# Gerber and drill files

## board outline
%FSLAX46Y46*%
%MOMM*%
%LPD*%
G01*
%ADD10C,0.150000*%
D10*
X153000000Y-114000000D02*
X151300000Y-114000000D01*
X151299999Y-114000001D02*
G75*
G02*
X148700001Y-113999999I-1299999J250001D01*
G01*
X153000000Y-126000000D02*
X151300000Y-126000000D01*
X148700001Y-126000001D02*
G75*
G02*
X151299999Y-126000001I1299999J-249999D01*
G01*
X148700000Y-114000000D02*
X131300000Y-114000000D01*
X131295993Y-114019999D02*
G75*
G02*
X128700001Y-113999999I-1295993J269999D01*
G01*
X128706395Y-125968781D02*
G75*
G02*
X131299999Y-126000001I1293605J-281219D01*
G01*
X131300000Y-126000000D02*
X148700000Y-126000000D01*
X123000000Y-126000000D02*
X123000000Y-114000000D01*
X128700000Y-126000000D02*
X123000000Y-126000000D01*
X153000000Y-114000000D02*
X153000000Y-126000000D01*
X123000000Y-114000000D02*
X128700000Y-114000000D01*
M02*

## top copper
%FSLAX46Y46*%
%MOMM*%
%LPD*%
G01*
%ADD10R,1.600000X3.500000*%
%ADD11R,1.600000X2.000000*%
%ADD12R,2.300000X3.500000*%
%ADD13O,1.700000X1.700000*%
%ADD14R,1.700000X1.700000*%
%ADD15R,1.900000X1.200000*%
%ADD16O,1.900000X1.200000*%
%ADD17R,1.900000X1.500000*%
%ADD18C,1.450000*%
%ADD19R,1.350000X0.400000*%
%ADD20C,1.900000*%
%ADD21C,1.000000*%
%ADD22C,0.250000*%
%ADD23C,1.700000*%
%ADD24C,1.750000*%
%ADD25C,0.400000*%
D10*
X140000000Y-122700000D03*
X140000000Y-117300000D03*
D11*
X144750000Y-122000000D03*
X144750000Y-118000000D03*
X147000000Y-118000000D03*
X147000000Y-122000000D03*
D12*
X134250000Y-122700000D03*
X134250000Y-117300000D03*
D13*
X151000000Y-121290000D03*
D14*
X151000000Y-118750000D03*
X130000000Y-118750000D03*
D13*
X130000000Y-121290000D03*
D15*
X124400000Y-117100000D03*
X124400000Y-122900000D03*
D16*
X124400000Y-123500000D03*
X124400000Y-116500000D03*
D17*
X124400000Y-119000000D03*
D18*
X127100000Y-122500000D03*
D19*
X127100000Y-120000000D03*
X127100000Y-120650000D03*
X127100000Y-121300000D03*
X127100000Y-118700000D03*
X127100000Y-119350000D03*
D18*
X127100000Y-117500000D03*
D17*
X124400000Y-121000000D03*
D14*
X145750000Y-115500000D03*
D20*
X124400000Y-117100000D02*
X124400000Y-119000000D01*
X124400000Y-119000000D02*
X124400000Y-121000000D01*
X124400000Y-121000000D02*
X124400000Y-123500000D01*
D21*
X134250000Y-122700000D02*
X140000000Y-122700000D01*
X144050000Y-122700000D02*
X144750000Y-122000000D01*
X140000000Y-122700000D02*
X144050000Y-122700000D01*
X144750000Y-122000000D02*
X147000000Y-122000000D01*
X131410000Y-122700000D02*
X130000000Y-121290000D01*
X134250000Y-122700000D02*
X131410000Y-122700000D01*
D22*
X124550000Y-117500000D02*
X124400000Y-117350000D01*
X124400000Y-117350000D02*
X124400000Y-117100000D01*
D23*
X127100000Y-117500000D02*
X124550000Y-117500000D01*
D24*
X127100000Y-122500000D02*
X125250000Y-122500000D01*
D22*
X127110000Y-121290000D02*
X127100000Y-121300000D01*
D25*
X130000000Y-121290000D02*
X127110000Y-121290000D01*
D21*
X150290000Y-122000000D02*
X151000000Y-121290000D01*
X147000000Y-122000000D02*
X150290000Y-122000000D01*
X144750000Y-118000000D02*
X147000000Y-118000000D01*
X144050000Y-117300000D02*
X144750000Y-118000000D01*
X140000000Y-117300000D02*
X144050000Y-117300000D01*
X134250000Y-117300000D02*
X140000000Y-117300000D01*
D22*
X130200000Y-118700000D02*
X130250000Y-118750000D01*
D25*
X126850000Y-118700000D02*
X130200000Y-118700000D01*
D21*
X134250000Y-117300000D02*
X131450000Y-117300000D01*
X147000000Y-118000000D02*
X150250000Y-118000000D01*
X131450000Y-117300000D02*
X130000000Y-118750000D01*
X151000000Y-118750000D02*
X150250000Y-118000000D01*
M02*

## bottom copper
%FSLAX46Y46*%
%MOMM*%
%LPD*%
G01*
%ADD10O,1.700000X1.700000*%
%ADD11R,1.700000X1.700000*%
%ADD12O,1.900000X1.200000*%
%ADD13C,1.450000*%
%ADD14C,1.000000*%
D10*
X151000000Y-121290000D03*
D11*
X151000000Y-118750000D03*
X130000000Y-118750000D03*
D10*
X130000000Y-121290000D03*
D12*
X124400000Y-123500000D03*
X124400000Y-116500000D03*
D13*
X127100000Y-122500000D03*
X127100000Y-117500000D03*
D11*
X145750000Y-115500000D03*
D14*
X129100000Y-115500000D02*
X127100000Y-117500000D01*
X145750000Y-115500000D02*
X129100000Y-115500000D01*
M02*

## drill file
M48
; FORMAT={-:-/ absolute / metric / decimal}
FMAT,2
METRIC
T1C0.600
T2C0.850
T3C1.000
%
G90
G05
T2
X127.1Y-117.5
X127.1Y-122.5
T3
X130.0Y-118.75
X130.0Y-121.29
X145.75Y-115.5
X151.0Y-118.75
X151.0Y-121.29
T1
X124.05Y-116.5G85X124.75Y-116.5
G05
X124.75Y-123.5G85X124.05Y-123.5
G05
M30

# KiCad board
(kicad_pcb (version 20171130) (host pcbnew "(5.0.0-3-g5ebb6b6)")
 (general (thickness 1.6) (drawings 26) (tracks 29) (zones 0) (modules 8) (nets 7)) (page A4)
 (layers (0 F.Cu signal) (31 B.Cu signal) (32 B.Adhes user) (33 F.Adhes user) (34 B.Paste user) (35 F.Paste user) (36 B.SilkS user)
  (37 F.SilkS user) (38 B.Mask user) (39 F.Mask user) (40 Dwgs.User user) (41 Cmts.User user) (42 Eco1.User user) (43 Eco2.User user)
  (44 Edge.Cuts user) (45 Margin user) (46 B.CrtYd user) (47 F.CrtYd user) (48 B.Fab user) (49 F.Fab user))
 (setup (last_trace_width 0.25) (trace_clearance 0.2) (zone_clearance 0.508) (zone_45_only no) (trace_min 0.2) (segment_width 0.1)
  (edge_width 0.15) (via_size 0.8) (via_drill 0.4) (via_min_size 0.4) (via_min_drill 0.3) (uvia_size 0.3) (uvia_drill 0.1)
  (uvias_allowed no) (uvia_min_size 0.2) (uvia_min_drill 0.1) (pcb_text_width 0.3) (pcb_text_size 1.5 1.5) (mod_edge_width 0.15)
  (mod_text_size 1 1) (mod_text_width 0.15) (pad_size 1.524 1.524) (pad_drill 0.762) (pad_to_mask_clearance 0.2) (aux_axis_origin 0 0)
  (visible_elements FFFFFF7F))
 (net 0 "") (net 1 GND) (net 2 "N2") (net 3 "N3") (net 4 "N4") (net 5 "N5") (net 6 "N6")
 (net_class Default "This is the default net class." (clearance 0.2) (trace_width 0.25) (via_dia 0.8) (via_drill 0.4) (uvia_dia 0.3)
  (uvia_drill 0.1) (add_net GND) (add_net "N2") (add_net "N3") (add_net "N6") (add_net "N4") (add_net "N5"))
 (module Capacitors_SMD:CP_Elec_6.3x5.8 (layer F.Cu) (at 140 120 270)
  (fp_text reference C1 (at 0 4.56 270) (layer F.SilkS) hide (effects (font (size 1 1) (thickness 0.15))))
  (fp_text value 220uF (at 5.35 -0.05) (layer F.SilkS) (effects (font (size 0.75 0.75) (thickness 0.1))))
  (pad 2 smd rect (at 2.7 0 90) (size 3.5 1.6) (layers F.Cu F.Paste F.Mask) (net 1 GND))
  (pad 1 smd rect (at -2.7 0 90) (size 3.5 1.6) (layers F.Cu F.Paste F.Mask) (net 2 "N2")))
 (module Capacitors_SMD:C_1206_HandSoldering (layer F.Cu) (at 144.75 120 270)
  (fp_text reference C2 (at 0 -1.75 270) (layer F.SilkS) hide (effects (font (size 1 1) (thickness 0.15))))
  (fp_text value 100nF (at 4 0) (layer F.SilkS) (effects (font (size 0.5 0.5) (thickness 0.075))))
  (pad 2 smd rect (at 2 0 270) (size 2 1.6) (layers F.Cu F.Paste F.Mask) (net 1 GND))
  (pad 1 smd rect (at -2 0 270) (size 2 1.6) (layers F.Cu F.Paste F.Mask) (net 2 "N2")))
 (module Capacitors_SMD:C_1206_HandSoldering (layer F.Cu) (at 147 120 270)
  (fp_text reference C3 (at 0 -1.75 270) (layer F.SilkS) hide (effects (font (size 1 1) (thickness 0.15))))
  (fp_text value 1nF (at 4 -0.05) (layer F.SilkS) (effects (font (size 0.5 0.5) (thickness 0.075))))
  (pad 1 smd rect (at -2 0 270) (size 2 1.6) (layers F.Cu F.Paste F.Mask) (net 2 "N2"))
  (pad 2 smd rect (at 2 0 270) (size 2 1.6) (layers F.Cu F.Paste F.Mask) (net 1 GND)))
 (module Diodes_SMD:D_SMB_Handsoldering (layer F.Cu) (at 134.25 120 270)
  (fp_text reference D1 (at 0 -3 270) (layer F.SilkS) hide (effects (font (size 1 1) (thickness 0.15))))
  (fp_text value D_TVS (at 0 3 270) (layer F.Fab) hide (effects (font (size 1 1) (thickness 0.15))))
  (pad 2 smd rect (at 2.7 0 270) (size 3.5 2.3) (layers F.Cu F.Paste F.Mask) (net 1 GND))
  (pad 1 smd rect (at -2.7 0 270) (size 3.5 2.3) (layers F.Cu F.Paste F.Mask) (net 2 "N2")))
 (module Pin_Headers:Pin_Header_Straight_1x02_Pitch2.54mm (layer F.Cu) (at 151 118.75)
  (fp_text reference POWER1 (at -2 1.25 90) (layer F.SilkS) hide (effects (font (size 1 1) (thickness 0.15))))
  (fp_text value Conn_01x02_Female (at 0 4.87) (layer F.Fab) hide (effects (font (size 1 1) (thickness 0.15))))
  (pad 2 thru_hole oval (at 0 2.54) (size 1.7 1.7) (drill 1) (layers *.Cu *.Mask) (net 1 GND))
  (pad 1 thru_hole rect (at 0 0) (size 1.7 1.7) (drill 1) (layers *.Cu *.Mask) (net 2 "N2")))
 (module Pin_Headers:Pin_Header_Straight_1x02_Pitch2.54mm (layer F.Cu) (at 130 118.75)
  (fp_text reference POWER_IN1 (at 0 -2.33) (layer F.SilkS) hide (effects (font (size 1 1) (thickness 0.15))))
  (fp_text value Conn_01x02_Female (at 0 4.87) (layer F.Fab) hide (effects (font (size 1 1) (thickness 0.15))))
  (pad 1 thru_hole rect (at 0 0) (size 1.7 1.7) (drill 1) (layers *.Cu *.Mask) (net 2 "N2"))
  (pad 2 thru_hole oval (at 0 2.54) (size 1.7 1.7) (drill 1) (layers *.Cu *.Mask) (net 1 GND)))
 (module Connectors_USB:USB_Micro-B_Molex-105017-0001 (layer F.Cu) (at 124.75 120 270)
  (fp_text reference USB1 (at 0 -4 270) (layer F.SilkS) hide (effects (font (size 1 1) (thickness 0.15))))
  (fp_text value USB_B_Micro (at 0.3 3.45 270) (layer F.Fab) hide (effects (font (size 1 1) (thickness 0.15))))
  (pad 6 smd rect (at -2.9 0.35 270) (size 1.2 1.9) (layers F.Cu F.Mask) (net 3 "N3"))
  (pad 6 smd rect (at 2.9 0.35 270) (size 1.2 1.9) (layers F.Cu F.Mask) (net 3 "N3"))
  (pad 6 thru_hole oval (at 3.5 0.35 270) (size 1.2 1.9) (drill oval 0.6 1.3) (layers *.Cu *.Mask) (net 3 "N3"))
  (pad 6 thru_hole oval (at -3.5 0.35 90) (size 1.2 1.9) (drill oval 0.6 1.3) (layers *.Cu *.Mask) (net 3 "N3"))
  (pad 6 smd rect (at -1 0.35 270) (size 1.5 1.9) (layers F.Cu F.Paste F.Mask) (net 3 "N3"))
  (pad 6 thru_hole circle (at 2.5 -2.35 270) (size 1.45 1.45) (drill 0.85) (layers *.Cu *.Mask) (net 3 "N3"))
  (pad 3 smd rect (at 0 -2.35 270) (size 0.4 1.35) (layers F.Cu F.Paste F.Mask) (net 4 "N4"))
  (pad 4 smd rect (at 0.65 -2.35 270) (size 0.4 1.35) (layers F.Cu F.Paste F.Mask) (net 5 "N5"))
  (pad 5 smd rect (at 1.3 -2.35 270) (size 0.4 1.35) (layers F.Cu F.Paste F.Mask) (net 1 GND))
  (pad 1 smd rect (at -1.3 -2.35 270) (size 0.4 1.35) (layers F.Cu F.Paste F.Mask) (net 2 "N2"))
  (pad 2 smd rect (at -0.65 -2.35 270) (size 0.4 1.35) (layers F.Cu F.Paste F.Mask) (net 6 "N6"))
  (pad 6 thru_hole circle (at -2.5 -2.35 270) (size 1.45 1.45) (drill 0.85) (layers *.Cu *.Mask) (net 3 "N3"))
  (pad 6 smd rect (at 1 0.35 270) (size 1.5 1.9) (layers F.Cu F.Paste F.Mask) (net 3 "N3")))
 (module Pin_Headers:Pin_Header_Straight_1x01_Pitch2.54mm (layer F.Cu) (at 145.75 115.5)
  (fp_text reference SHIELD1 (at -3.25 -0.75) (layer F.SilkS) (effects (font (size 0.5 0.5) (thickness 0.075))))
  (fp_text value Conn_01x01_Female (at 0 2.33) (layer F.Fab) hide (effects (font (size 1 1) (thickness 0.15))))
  (pad 1 thru_hole rect (at 0 0) (size 1.7 1.7) (drill 1) (layers *.Cu *.Mask) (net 3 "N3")))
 (gr_line (start 153 114) (end 151.3 114) (layer Edge.Cuts) (width 0.15))
 (gr_arc (start 150 113.75) (end 148.700001 113.999999) (angle -158.2289459) (layer Edge.Cuts) (width 0.15))
 (gr_line (start 153 126) (end 151.3 126) (layer Edge.Cuts) (width 0.15))
 (gr_arc (start 150 126.25) (end 151.299999 126.000001) (angle -158.2290064) (layer Edge.Cuts) (width 0.15))
 (gr_line (start 148.7 114) (end 131.3 114) (layer Edge.Cuts) (width 0.15))
 (gr_arc (start 130 113.75) (end 128.700001 113.999999) (angle -157.346184) (layer Edge.Cuts) (width 0.15))
 (gr_arc (start 130 126.25) (end 131.299999 126.000001) (angle -156.8496992) (layer Edge.Cuts) (width 0.15))
 (gr_line (start 131.3 126) (end 148.7 126) (layer Edge.Cuts) (width 0.15))
 (gr_line (start 123 126) (end 123 114) (layer Edge.Cuts) (width 0.15))
 (gr_line (start 128.7 126) (end 123 126) (layer Edge.Cuts) (width 0.15))
 (gr_line (start 153 114) (end 153 126) (layer Edge.Cuts) (width 0.15))
 (gr_line (start 123 114) (end 128.7 114) (layer Edge.Cuts) (width 0.15))
 (segment (start 124.4 117.1) (end 124.4 119) (width 1.9) (layer F.Cu) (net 3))
 (segment (start 124.4 119) (end 124.4 121) (width 1.9) (layer F.Cu) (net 3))
 (segment (start 124.4 121) (end 124.4 123.5) (width 1.9) (layer F.Cu) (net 3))
 (segment (start 134.25 122.7) (end 140 122.7) (width 1) (layer F.Cu) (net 1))
 (segment (start 144.05 122.7) (end 144.75 122) (width 1) (layer F.Cu) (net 1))
 (segment (start 140 122.7) (end 144.05 122.7) (width 1) (layer F.Cu) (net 1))
 (segment (start 144.75 122) (end 147 122) (width 1) (layer F.Cu) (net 1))
 (segment (start 131.41 122.7) (end 130 121.29) (width 1) (layer F.Cu) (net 1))
 (segment (start 134.25 122.7) (end 131.41 122.7) (width 1) (layer F.Cu) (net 1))
 (segment (start 124.55 117.5) (end 124.4 117.35) (width 0.25) (layer F.Cu) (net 3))
 (segment (start 124.4 117.35) (end 124.4 117.1) (width 0.25) (layer F.Cu) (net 3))
 (segment (start 127.1 117.5) (end 124.55 117.5) (width 1.7) (layer F.Cu) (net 3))
 (segment (start 127.1 122.5) (end 125.25 122.5) (width 1.75) (layer F.Cu) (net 3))
 (segment (start 127.11 121.29) (end 127.1 121.3) (width 0.25) (layer F.Cu) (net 1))
 (segment (start 130 121.29) (end 127.11 121.29) (width 0.4) (layer F.Cu) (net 1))
 (segment (start 150.29 122) (end 151 121.29) (width 1) (layer F.Cu) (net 1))
 (segment (start 147 122) (end 150.29 122) (width 1) (layer F.Cu) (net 1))
 (segment (start 144.75 118) (end 147 118) (width 1) (layer F.Cu) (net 2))
 (segment (start 144.05 117.3) (end 144.75 118) (width 1) (layer F.Cu) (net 2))
 (segment (start 140 117.3) (end 144.05 117.3) (width 1) (layer F.Cu) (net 2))
 (segment (start 134.25 117.3) (end 140 117.3) (width 1) (layer F.Cu) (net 2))
 (segment (start 130.2 118.7) (end 130.25 118.75) (width 0.25) (layer F.Cu) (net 2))
 (segment (start 126.85 118.7) (end 130.2 118.7) (width 0.4) (layer F.Cu) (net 2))
 (segment (start 134.25 117.3) (end 131.45 117.3) (width 1) (layer F.Cu) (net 2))
 (segment (start 147 118) (end 150.25 118) (width 1) (layer F.Cu) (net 2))
 (segment (start 131.45 117.3) (end 130 118.75) (width 1) (layer F.Cu) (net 2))
 (segment (start 151 118.75) (end 150.25 118) (width 1) (layer F.Cu) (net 2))
 (segment (start 129.1 115.5) (end 127.1 117.5) (width 1) (layer B.Cu) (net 3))
 (segment (start 145.75 115.5) (end 129.1 115.5) (width 1) (layer B.Cu) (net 3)))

